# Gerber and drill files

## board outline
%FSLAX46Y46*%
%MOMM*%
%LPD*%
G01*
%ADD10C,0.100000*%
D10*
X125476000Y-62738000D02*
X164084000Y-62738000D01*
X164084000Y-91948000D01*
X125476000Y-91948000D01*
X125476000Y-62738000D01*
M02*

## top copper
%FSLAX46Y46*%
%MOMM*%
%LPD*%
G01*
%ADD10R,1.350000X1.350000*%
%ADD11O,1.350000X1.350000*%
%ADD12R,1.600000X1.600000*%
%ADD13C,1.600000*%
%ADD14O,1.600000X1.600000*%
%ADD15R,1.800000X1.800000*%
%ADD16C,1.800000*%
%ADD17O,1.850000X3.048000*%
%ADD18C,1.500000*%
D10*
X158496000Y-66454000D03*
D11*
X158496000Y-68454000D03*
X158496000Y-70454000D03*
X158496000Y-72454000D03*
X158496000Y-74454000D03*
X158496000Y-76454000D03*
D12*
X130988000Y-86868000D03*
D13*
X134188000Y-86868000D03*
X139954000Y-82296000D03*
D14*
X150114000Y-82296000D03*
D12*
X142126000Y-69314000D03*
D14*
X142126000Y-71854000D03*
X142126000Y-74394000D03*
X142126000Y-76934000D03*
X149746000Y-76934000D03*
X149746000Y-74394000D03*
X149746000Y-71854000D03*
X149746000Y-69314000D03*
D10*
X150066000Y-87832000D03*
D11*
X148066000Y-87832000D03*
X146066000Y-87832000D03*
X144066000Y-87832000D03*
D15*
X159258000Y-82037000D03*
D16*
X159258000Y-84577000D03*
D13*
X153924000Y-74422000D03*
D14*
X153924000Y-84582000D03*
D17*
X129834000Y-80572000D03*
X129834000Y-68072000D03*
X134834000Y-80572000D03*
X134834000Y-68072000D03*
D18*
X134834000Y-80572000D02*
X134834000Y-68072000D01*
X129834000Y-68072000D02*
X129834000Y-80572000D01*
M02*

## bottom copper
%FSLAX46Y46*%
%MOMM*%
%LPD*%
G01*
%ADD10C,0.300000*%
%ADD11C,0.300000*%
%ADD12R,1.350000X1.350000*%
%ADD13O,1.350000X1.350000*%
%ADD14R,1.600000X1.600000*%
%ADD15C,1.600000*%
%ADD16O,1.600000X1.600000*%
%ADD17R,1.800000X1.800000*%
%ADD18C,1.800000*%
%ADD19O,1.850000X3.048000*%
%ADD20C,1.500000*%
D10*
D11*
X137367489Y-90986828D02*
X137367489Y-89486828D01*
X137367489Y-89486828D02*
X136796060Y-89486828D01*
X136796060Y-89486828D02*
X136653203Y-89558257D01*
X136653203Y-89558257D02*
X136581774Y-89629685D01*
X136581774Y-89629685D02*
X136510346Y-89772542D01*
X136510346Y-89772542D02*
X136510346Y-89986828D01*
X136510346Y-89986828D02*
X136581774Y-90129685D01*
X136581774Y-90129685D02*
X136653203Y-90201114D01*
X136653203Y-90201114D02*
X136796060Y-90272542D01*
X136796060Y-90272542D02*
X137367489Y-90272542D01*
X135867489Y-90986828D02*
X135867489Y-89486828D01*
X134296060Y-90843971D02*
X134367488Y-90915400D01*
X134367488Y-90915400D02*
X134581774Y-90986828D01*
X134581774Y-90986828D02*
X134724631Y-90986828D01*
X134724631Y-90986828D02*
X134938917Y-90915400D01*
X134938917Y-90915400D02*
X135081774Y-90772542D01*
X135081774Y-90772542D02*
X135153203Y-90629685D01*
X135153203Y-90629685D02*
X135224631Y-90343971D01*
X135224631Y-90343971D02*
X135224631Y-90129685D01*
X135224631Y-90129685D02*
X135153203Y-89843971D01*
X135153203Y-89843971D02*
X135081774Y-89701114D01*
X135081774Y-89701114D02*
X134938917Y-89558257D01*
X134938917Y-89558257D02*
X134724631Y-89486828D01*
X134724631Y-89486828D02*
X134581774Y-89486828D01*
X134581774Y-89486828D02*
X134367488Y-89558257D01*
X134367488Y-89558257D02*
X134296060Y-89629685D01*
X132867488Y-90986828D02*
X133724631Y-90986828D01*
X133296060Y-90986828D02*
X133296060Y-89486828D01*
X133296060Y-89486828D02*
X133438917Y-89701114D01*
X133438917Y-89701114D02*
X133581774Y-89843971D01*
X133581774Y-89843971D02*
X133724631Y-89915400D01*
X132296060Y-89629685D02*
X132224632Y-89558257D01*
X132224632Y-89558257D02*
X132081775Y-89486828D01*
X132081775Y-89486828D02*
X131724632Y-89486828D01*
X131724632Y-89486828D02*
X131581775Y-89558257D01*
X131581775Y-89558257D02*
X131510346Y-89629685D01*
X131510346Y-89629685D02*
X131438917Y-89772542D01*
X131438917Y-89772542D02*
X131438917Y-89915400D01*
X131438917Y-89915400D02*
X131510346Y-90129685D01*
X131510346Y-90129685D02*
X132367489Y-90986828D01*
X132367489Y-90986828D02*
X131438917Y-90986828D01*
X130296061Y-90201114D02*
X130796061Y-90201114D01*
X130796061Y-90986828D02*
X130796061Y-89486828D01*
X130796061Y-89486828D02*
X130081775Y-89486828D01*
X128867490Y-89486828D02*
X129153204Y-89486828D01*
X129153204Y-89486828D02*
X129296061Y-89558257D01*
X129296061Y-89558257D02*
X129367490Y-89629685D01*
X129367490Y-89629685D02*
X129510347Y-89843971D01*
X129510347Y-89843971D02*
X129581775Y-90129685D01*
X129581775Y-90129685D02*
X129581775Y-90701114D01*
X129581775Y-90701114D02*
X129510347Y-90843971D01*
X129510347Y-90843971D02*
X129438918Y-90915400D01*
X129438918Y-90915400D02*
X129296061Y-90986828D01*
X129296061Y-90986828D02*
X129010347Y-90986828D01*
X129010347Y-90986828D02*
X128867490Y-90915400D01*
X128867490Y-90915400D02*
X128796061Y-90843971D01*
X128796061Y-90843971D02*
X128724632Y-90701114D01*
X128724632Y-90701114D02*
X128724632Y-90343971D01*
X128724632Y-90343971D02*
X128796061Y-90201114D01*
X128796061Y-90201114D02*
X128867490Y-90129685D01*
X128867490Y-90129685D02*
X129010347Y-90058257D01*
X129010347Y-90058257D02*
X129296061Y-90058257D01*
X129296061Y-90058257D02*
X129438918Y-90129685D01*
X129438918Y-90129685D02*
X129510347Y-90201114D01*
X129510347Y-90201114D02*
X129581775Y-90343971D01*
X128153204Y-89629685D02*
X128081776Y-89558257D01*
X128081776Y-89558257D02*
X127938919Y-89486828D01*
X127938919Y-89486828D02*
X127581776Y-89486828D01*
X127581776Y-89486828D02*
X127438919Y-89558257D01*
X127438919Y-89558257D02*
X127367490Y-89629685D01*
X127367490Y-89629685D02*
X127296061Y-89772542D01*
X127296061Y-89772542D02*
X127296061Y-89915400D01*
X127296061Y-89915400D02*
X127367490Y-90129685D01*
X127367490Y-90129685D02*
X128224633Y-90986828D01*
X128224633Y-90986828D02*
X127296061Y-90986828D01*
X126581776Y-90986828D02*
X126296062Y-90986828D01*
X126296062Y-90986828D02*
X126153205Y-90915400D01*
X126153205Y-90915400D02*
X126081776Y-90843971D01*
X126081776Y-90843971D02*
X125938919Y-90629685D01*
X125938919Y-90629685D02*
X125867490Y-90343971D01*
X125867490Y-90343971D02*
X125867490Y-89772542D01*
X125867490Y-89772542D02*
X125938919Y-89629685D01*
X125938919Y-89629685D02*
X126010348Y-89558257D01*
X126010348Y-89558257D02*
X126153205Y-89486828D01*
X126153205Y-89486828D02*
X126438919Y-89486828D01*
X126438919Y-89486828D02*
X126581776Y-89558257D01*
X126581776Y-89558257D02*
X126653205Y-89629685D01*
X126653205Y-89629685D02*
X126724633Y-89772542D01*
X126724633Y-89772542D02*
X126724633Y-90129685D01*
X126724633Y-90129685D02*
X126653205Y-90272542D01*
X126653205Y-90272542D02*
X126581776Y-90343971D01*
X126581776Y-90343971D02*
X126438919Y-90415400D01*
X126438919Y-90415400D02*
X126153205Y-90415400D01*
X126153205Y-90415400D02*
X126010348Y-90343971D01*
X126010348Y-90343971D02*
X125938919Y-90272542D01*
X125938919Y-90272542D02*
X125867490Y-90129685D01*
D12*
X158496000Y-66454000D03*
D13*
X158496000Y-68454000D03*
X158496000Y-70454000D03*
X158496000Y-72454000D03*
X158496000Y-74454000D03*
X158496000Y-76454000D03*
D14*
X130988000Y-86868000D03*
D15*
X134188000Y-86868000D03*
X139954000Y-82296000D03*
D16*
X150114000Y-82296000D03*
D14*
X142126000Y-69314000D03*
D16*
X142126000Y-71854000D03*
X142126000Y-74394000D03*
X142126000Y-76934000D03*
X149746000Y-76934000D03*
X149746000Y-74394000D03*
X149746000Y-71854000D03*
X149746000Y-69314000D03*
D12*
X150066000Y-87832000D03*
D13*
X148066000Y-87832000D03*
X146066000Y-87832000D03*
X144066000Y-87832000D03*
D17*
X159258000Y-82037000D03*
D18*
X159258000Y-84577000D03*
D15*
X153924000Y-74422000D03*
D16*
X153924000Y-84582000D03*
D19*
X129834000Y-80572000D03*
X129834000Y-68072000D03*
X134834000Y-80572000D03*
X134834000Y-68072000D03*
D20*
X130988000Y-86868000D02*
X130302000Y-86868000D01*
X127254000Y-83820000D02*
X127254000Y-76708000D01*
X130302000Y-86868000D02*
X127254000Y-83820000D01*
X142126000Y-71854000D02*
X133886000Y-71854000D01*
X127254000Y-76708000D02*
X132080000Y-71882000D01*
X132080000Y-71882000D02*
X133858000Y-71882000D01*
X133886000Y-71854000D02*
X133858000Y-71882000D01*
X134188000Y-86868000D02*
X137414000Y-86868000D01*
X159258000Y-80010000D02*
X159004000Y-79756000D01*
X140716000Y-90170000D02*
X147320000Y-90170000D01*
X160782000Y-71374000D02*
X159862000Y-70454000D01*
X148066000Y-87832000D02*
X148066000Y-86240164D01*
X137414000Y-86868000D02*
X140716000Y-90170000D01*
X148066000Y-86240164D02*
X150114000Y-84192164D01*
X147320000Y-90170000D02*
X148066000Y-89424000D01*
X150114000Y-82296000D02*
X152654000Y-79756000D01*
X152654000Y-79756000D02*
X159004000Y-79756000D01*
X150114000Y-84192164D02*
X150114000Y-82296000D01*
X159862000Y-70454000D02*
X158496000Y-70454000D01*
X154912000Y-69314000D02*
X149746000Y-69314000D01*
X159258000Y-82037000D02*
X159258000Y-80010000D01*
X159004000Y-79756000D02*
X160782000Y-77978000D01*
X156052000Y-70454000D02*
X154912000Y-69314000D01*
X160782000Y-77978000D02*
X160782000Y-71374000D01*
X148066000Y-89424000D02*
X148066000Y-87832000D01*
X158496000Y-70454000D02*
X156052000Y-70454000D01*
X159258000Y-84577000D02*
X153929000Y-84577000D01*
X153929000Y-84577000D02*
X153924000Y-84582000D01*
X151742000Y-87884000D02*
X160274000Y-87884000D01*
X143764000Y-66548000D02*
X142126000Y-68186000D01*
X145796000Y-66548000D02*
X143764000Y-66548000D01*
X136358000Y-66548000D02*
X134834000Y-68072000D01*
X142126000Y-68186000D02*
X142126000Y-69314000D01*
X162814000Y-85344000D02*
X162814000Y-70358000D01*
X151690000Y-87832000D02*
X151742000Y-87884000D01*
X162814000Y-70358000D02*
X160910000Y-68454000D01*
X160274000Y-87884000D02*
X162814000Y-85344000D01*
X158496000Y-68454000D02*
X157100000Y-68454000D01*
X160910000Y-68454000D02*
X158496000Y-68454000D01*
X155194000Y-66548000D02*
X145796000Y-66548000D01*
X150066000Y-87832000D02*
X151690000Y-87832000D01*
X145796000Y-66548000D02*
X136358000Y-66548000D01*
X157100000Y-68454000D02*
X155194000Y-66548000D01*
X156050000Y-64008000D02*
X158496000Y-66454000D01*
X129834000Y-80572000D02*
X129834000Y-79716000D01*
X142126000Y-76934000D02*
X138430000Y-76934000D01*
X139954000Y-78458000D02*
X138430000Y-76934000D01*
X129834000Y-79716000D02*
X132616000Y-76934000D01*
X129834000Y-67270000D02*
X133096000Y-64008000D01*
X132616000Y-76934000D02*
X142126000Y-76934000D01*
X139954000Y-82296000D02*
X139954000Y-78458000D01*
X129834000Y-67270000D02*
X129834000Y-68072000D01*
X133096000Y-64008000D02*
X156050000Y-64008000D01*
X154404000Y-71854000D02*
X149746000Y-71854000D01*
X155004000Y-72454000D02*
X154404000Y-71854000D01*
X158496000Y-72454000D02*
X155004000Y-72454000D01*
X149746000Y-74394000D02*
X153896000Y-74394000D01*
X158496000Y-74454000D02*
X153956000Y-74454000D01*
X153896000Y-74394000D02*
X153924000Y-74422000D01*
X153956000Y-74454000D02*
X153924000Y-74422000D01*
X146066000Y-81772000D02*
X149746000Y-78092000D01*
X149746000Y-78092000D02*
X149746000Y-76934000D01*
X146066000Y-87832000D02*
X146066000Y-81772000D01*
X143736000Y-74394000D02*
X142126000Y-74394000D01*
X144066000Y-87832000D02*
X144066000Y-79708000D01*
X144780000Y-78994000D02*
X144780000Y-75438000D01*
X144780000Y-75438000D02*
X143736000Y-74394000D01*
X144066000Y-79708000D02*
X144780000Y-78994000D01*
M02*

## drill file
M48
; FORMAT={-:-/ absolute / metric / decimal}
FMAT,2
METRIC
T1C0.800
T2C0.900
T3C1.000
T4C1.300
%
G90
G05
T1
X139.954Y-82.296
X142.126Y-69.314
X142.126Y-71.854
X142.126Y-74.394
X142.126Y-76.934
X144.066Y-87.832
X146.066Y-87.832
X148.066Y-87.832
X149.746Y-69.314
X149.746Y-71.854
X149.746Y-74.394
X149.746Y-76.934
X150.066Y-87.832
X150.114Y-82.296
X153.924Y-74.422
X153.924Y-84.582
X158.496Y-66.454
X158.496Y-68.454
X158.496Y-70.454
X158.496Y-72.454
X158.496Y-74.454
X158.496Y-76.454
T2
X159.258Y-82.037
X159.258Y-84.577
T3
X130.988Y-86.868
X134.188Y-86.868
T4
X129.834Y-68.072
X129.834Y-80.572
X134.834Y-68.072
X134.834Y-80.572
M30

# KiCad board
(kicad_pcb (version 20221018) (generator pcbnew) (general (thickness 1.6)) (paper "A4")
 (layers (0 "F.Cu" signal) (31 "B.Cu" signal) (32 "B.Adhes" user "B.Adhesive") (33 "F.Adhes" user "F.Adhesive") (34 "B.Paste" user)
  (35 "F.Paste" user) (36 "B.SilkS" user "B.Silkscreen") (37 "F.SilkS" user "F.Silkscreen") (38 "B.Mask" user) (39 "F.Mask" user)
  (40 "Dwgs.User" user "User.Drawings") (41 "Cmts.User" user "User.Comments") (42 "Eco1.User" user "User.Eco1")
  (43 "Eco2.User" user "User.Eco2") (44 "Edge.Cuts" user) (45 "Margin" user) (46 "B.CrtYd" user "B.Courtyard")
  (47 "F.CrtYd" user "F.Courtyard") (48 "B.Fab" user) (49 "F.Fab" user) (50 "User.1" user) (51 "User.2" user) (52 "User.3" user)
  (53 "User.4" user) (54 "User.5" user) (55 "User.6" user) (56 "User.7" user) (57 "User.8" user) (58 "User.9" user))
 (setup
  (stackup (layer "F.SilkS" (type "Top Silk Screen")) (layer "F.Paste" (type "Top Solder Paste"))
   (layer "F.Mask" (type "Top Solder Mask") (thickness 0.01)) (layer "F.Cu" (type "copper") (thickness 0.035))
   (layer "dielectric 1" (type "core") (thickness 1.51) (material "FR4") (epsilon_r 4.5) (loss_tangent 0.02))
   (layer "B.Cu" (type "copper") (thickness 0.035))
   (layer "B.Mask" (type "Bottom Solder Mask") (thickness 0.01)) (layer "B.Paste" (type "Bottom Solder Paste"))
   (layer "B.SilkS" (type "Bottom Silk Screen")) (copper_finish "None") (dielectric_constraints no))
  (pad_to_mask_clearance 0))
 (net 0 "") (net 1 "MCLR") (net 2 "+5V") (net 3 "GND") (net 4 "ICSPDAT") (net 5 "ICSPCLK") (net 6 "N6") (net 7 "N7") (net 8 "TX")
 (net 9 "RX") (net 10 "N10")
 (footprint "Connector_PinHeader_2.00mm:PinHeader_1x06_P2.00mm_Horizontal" (layer "F.Cu") (at 158.496 66.454)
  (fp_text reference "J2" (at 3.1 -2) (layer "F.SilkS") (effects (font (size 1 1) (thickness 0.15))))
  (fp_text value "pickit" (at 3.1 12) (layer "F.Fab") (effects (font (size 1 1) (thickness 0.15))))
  (pad "1" thru_hole rect (at 0 0) (size 1.35 1.35) (drill 0.8) (layers "*.Cu" "*.Mask") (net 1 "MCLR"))
  (pad "2" thru_hole oval (at 0 2) (size 1.35 1.35) (drill 0.8) (layers "*.Cu" "*.Mask") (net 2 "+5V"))
  (pad "3" thru_hole oval (at 0 4) (size 1.35 1.35) (drill 0.8) (layers "*.Cu" "*.Mask") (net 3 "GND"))
  (pad "4" thru_hole oval (at 0 6) (size 1.35 1.35) (drill 0.8) (layers "*.Cu" "*.Mask") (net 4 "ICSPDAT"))
  (pad "5" thru_hole oval (at 0 8) (size 1.35 1.35) (drill 0.8) (layers "*.Cu" "*.Mask") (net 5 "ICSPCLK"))
  (pad "6" thru_hole oval (at 0 10) (size 1.35 1.35) (drill 0.8) (layers "*.Cu" "*.Mask") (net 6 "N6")))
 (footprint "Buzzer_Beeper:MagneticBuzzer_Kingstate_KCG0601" (layer "F.Cu") (at 130.988 86.868)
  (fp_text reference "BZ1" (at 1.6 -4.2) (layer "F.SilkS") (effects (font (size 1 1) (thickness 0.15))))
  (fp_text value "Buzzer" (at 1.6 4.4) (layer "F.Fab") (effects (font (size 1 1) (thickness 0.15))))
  (pad "1" thru_hole rect (at 0 0) (size 1.6 1.6) (drill 1) (layers "*.Cu" "*.Mask") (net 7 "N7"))
  (pad "2" thru_hole circle (at 3.2 0) (size 1.6 1.6) (drill 1) (layers "*.Cu" "*.Mask") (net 3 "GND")))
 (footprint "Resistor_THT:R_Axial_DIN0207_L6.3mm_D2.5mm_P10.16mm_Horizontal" (layer "F.Cu") (at 139.954 82.296)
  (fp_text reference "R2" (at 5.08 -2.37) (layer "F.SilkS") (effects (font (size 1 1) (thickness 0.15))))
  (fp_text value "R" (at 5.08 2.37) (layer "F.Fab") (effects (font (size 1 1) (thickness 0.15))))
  (pad "1" thru_hole circle (at 0 0) (size 1.6 1.6) (drill 0.8) (layers "*.Cu" "*.Mask") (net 1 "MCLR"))
  (pad "2" thru_hole oval (at 10.16 0) (size 1.6 1.6) (drill 0.8) (layers "*.Cu" "*.Mask") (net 3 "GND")))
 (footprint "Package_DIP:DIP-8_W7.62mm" (layer "F.Cu") (at 142.126 69.314)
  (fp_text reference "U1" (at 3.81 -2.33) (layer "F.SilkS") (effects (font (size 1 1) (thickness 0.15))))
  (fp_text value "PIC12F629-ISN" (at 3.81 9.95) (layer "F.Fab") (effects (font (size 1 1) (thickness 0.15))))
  (pad "1" thru_hole rect (at 0 0) (size 1.6 1.6) (drill 0.8) (layers "*.Cu" "*.Mask") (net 2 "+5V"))
  (pad "2" thru_hole oval (at 0 2.54) (size 1.6 1.6) (drill 0.8) (layers "*.Cu" "*.Mask") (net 7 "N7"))
  (pad "3" thru_hole oval (at 0 5.08) (size 1.6 1.6) (drill 0.8) (layers "*.Cu" "*.Mask") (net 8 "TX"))
  (pad "4" thru_hole oval (at 0 7.62) (size 1.6 1.6) (drill 0.8) (layers "*.Cu" "*.Mask") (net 1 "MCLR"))
  (pad "5" thru_hole oval (at 7.62 7.62) (size 1.6 1.6) (drill 0.8) (layers "*.Cu" "*.Mask") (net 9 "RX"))
  (pad "6" thru_hole oval (at 7.62 5.08) (size 1.6 1.6) (drill 0.8) (layers "*.Cu" "*.Mask") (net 5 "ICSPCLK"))
  (pad "7" thru_hole oval (at 7.62 2.54) (size 1.6 1.6) (drill 0.8) (layers "*.Cu" "*.Mask") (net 4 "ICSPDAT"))
  (pad "8" thru_hole oval (at 7.62 0) (size 1.6 1.6) (drill 0.8) (layers "*.Cu" "*.Mask") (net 3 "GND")))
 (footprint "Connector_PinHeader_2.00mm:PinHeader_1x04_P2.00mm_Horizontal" (layer "F.Cu") (at 150.066 87.832 -90)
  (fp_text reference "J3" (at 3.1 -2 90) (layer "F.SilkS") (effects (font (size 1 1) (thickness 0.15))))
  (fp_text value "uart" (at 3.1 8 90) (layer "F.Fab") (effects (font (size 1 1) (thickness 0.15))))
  (pad "1" thru_hole rect (at 0 0 270) (size 1.35 1.35) (drill 0.8) (layers "*.Cu" "*.Mask") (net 2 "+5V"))
  (pad "2" thru_hole oval (at 0 2 270) (size 1.35 1.35) (drill 0.8) (layers "*.Cu" "*.Mask") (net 3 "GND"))
  (pad "3" thru_hole oval (at 0 4 270) (size 1.35 1.35) (drill 0.8) (layers "*.Cu" "*.Mask") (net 9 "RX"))
  (pad "4" thru_hole oval (at 0 6 270) (size 1.35 1.35) (drill 0.8) (layers "*.Cu" "*.Mask") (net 8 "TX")))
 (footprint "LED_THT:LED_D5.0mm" (layer "F.Cu") (at 159.258 82.037 -90)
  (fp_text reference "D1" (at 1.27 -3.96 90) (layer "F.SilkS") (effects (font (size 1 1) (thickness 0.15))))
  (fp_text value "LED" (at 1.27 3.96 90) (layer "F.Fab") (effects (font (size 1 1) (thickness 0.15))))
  (pad "1" thru_hole rect (at 0 0 270) (size 1.8 1.8) (drill 0.9) (layers "*.Cu" "*.Mask") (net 3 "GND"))
  (pad "2" thru_hole circle (at 2.54 0 270) (size 1.8 1.8) (drill 0.9) (layers "*.Cu" "*.Mask") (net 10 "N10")))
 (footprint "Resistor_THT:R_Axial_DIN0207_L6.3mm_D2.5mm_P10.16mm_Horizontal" (layer "F.Cu") (at 153.924 74.422 -90)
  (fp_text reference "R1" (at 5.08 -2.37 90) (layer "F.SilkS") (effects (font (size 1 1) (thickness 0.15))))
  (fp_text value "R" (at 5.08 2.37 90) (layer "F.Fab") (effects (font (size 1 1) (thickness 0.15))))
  (pad "1" thru_hole circle (at 0 0 270) (size 1.6 1.6) (drill 0.8) (layers "*.Cu" "*.Mask") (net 5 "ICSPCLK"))
  (pad "2" thru_hole oval (at 10.16 0 270) (size 1.6 1.6) (drill 0.8) (layers "*.Cu" "*.Mask") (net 10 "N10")))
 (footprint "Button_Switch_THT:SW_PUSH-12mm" (layer "F.Cu") (at 129.834 80.572 90)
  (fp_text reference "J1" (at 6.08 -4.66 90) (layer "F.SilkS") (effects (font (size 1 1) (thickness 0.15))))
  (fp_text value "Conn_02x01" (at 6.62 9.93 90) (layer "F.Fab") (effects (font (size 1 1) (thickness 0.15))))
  (pad "1" thru_hole oval (at 0 0 90) (size 3.048 1.85) (drill 1.3) (layers "*.Cu" "*.Mask") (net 1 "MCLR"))
  (pad "1" thru_hole oval (at 12.5 0 90) (size 3.048 1.85) (drill 1.3) (layers "*.Cu" "*.Mask") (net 1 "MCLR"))
  (pad "2" thru_hole oval (at 0 5 90) (size 3.048 1.85) (drill 1.3) (layers "*.Cu" "*.Mask") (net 2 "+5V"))
  (pad "2" thru_hole oval (at 12.5 5 90) (size 3.048 1.85) (drill 1.3) (layers "*.Cu" "*.Mask") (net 2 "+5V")))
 (gr_rect (start 125.476 62.738) (end 164.084 91.948) (stroke (width 0.1) (type default)) (fill none) (layer "Edge.Cuts"))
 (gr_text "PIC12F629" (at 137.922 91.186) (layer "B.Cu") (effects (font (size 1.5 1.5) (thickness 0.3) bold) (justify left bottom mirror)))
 (segment (start 130.988 86.868) (end 130.302 86.868) (width 1.5) (layer "B.Cu") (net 7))
 (segment (start 127.254 83.82) (end 127.254 76.708) (width 1.5) (layer "B.Cu") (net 7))
 (segment (start 130.302 86.868) (end 127.254 83.82) (width 1.5) (layer "B.Cu") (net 7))
 (segment (start 142.126 71.854) (end 133.886 71.854) (width 1.5) (layer "B.Cu") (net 7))
 (segment (start 127.254 76.708) (end 132.08 71.882) (width 1.5) (layer "B.Cu") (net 7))
 (segment (start 132.08 71.882) (end 133.858 71.882) (width 1.5) (layer "B.Cu") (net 7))
 (segment (start 133.886 71.854) (end 133.858 71.882) (width 1.5) (layer "B.Cu") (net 7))
 (segment (start 134.188 86.868) (end 137.414 86.868) (width 1.5) (layer "B.Cu") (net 3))
 (segment (start 159.258 80.01) (end 159.004 79.756) (width 1.5) (layer "B.Cu") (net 3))
 (segment (start 140.716 90.17) (end 147.32 90.17) (width 1.5) (layer "B.Cu") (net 3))
 (segment (start 160.782 71.374) (end 159.862 70.454) (width 1.5) (layer "B.Cu") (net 3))
 (segment (start 148.066 87.832) (end 148.066 86.240164) (width 1.5) (layer "B.Cu") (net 3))
 (segment (start 137.414 86.868) (end 140.716 90.17) (width 1.5) (layer "B.Cu") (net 3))
 (segment (start 148.066 86.240164) (end 150.114 84.192164) (width 1.5) (layer "B.Cu") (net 3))
 (segment (start 147.32 90.17) (end 148.066 89.424) (width 1.5) (layer "B.Cu") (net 3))
 (segment (start 150.114 82.296) (end 152.654 79.756) (width 1.5) (layer "B.Cu") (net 3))
 (segment (start 152.654 79.756) (end 159.004 79.756) (width 1.5) (layer "B.Cu") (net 3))
 (segment (start 150.114 84.192164) (end 150.114 82.296) (width 1.5) (layer "B.Cu") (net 3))
 (segment (start 159.862 70.454) (end 158.496 70.454) (width 1.5) (layer "B.Cu") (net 3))
 (segment (start 154.912 69.314) (end 149.746 69.314) (width 1.5) (layer "B.Cu") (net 3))
 (segment (start 159.258 82.037) (end 159.258 80.01) (width 1.5) (layer "B.Cu") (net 3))
 (segment (start 159.004 79.756) (end 160.782 77.978) (width 1.5) (layer "B.Cu") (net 3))
 (segment (start 156.052 70.454) (end 154.912 69.314) (width 1.5) (layer "B.Cu") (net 3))
 (segment (start 160.782 77.978) (end 160.782 71.374) (width 1.5) (layer "B.Cu") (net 3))
 (segment (start 148.066 89.424) (end 148.066 87.832) (width 1.5) (layer "B.Cu") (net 3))
 (segment (start 158.496 70.454) (end 156.052 70.454) (width 1.5) (layer "B.Cu") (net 3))
 (segment (start 159.258 84.577) (end 153.929 84.577) (width 1.5) (layer "B.Cu") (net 10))
 (segment (start 153.929 84.577) (end 153.924 84.582) (width 1.5) (layer "B.Cu") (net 10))
 (segment (start 134.834 80.572) (end 134.834 68.072) (width 1.5) (layer "F.Cu") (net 2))
 (segment (start 151.742 87.884) (end 160.274 87.884) (width 1.5) (layer "B.Cu") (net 2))
 (segment (start 143.764 66.548) (end 142.126 68.186) (width 1.5) (layer "B.Cu") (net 2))
 (segment (start 145.796 66.548) (end 143.764 66.548) (width 1.5) (layer "B.Cu") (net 2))
 (segment (start 136.358 66.548) (end 134.834 68.072) (width 1.5) (layer "B.Cu") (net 2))
 (segment (start 142.126 68.186) (end 142.126 69.314) (width 1.5) (layer "B.Cu") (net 2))
 (segment (start 162.814 85.344) (end 162.814 70.358) (width 1.5) (layer "B.Cu") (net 2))
 (segment (start 151.69 87.832) (end 151.742 87.884) (width 1.5) (layer "B.Cu") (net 2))
 (segment (start 162.814 70.358) (end 160.91 68.454) (width 1.5) (layer "B.Cu") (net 2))
 (segment (start 160.274 87.884) (end 162.814 85.344) (width 1.5) (layer "B.Cu") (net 2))
 (segment (start 158.496 68.454) (end 157.1 68.454) (width 1.5) (layer "B.Cu") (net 2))
 (segment (start 160.91 68.454) (end 158.496 68.454) (width 1.5) (layer "B.Cu") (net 2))
 (segment (start 155.194 66.548) (end 145.796 66.548) (width 1.5) (layer "B.Cu") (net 2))
 (segment (start 150.066 87.832) (end 151.69 87.832) (width 1.5) (layer "B.Cu") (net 2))
 (segment (start 145.796 66.548) (end 136.358 66.548) (width 1.5) (layer "B.Cu") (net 2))
 (segment (start 157.1 68.454) (end 155.194 66.548) (width 1.5) (layer "B.Cu") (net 2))
 (segment (start 129.834 68.072) (end 129.834 80.572) (width 1.5) (layer "F.Cu") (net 1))
 (segment (start 156.05 64.008) (end 158.496 66.454) (width 1.5) (layer "B.Cu") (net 1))
 (segment (start 129.834 80.572) (end 129.834 79.716) (width 1.5) (layer "B.Cu") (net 1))
 (segment (start 142.126 76.934) (end 138.43 76.934) (width 1.5) (layer "B.Cu") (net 1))
 (segment (start 139.954 78.458) (end 138.43 76.934) (width 1.5) (layer "B.Cu") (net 1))
 (segment (start 129.834 79.716) (end 132.616 76.934) (width 1.5) (layer "B.Cu") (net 1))
 (segment (start 129.834 67.27) (end 133.096 64.008) (width 1.5) (layer "B.Cu") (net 1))
 (segment (start 132.616 76.934) (end 142.126 76.934) (width 1.5) (layer "B.Cu") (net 1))
 (segment (start 139.954 82.296) (end 139.954 78.458) (width 1.5) (layer "B.Cu") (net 1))
 (segment (start 129.834 67.27) (end 129.834 68.072) (width 1.5) (layer "B.Cu") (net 1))
 (segment (start 133.096 64.008) (end 156.05 64.008) (width 1.5) (layer "B.Cu") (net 1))
 (segment (start 154.404 71.854) (end 149.746 71.854) (width 1.5) (layer "B.Cu") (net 4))
 (segment (start 155.004 72.454) (end 154.404 71.854) (width 1.5) (layer "B.Cu") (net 4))
 (segment (start 158.496 72.454) (end 155.004 72.454) (width 1.5) (layer "B.Cu") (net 4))
 (segment (start 149.746 74.394) (end 153.896 74.394) (width 1.5) (layer "B.Cu") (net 5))
 (segment (start 158.496 74.454) (end 153.956 74.454) (width 1.5) (layer "B.Cu") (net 5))
 (segment (start 153.896 74.394) (end 153.924 74.422) (width 1.5) (layer "B.Cu") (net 5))
 (segment (start 153.956 74.454) (end 153.924 74.422) (width 1.5) (layer "B.Cu") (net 5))
 (segment (start 146.066 81.772) (end 149.746 78.092) (width 1.5) (layer "B.Cu") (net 9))
 (segment (start 149.746 78.092) (end 149.746 76.934) (width 1.5) (layer "B.Cu") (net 9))
 (segment (start 146.066 87.832) (end 146.066 81.772) (width 1.5) (layer "B.Cu") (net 9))
 (segment (start 143.736 74.394) (end 142.126 74.394) (width 1.5) (layer "B.Cu") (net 8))
 (segment (start 144.066 87.832) (end 144.066 79.708) (width 1.5) (layer "B.Cu") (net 8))
 (segment (start 144.78 78.994) (end 144.78 75.438) (width 1.5) (layer "B.Cu") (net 8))
 (segment (start 144.78 75.438) (end 143.736 74.394) (width 1.5) (layer "B.Cu") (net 8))
 (segment (start 144.066 79.708) (end 144.78 78.994) (width 1.5) (layer "B.Cu") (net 8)))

